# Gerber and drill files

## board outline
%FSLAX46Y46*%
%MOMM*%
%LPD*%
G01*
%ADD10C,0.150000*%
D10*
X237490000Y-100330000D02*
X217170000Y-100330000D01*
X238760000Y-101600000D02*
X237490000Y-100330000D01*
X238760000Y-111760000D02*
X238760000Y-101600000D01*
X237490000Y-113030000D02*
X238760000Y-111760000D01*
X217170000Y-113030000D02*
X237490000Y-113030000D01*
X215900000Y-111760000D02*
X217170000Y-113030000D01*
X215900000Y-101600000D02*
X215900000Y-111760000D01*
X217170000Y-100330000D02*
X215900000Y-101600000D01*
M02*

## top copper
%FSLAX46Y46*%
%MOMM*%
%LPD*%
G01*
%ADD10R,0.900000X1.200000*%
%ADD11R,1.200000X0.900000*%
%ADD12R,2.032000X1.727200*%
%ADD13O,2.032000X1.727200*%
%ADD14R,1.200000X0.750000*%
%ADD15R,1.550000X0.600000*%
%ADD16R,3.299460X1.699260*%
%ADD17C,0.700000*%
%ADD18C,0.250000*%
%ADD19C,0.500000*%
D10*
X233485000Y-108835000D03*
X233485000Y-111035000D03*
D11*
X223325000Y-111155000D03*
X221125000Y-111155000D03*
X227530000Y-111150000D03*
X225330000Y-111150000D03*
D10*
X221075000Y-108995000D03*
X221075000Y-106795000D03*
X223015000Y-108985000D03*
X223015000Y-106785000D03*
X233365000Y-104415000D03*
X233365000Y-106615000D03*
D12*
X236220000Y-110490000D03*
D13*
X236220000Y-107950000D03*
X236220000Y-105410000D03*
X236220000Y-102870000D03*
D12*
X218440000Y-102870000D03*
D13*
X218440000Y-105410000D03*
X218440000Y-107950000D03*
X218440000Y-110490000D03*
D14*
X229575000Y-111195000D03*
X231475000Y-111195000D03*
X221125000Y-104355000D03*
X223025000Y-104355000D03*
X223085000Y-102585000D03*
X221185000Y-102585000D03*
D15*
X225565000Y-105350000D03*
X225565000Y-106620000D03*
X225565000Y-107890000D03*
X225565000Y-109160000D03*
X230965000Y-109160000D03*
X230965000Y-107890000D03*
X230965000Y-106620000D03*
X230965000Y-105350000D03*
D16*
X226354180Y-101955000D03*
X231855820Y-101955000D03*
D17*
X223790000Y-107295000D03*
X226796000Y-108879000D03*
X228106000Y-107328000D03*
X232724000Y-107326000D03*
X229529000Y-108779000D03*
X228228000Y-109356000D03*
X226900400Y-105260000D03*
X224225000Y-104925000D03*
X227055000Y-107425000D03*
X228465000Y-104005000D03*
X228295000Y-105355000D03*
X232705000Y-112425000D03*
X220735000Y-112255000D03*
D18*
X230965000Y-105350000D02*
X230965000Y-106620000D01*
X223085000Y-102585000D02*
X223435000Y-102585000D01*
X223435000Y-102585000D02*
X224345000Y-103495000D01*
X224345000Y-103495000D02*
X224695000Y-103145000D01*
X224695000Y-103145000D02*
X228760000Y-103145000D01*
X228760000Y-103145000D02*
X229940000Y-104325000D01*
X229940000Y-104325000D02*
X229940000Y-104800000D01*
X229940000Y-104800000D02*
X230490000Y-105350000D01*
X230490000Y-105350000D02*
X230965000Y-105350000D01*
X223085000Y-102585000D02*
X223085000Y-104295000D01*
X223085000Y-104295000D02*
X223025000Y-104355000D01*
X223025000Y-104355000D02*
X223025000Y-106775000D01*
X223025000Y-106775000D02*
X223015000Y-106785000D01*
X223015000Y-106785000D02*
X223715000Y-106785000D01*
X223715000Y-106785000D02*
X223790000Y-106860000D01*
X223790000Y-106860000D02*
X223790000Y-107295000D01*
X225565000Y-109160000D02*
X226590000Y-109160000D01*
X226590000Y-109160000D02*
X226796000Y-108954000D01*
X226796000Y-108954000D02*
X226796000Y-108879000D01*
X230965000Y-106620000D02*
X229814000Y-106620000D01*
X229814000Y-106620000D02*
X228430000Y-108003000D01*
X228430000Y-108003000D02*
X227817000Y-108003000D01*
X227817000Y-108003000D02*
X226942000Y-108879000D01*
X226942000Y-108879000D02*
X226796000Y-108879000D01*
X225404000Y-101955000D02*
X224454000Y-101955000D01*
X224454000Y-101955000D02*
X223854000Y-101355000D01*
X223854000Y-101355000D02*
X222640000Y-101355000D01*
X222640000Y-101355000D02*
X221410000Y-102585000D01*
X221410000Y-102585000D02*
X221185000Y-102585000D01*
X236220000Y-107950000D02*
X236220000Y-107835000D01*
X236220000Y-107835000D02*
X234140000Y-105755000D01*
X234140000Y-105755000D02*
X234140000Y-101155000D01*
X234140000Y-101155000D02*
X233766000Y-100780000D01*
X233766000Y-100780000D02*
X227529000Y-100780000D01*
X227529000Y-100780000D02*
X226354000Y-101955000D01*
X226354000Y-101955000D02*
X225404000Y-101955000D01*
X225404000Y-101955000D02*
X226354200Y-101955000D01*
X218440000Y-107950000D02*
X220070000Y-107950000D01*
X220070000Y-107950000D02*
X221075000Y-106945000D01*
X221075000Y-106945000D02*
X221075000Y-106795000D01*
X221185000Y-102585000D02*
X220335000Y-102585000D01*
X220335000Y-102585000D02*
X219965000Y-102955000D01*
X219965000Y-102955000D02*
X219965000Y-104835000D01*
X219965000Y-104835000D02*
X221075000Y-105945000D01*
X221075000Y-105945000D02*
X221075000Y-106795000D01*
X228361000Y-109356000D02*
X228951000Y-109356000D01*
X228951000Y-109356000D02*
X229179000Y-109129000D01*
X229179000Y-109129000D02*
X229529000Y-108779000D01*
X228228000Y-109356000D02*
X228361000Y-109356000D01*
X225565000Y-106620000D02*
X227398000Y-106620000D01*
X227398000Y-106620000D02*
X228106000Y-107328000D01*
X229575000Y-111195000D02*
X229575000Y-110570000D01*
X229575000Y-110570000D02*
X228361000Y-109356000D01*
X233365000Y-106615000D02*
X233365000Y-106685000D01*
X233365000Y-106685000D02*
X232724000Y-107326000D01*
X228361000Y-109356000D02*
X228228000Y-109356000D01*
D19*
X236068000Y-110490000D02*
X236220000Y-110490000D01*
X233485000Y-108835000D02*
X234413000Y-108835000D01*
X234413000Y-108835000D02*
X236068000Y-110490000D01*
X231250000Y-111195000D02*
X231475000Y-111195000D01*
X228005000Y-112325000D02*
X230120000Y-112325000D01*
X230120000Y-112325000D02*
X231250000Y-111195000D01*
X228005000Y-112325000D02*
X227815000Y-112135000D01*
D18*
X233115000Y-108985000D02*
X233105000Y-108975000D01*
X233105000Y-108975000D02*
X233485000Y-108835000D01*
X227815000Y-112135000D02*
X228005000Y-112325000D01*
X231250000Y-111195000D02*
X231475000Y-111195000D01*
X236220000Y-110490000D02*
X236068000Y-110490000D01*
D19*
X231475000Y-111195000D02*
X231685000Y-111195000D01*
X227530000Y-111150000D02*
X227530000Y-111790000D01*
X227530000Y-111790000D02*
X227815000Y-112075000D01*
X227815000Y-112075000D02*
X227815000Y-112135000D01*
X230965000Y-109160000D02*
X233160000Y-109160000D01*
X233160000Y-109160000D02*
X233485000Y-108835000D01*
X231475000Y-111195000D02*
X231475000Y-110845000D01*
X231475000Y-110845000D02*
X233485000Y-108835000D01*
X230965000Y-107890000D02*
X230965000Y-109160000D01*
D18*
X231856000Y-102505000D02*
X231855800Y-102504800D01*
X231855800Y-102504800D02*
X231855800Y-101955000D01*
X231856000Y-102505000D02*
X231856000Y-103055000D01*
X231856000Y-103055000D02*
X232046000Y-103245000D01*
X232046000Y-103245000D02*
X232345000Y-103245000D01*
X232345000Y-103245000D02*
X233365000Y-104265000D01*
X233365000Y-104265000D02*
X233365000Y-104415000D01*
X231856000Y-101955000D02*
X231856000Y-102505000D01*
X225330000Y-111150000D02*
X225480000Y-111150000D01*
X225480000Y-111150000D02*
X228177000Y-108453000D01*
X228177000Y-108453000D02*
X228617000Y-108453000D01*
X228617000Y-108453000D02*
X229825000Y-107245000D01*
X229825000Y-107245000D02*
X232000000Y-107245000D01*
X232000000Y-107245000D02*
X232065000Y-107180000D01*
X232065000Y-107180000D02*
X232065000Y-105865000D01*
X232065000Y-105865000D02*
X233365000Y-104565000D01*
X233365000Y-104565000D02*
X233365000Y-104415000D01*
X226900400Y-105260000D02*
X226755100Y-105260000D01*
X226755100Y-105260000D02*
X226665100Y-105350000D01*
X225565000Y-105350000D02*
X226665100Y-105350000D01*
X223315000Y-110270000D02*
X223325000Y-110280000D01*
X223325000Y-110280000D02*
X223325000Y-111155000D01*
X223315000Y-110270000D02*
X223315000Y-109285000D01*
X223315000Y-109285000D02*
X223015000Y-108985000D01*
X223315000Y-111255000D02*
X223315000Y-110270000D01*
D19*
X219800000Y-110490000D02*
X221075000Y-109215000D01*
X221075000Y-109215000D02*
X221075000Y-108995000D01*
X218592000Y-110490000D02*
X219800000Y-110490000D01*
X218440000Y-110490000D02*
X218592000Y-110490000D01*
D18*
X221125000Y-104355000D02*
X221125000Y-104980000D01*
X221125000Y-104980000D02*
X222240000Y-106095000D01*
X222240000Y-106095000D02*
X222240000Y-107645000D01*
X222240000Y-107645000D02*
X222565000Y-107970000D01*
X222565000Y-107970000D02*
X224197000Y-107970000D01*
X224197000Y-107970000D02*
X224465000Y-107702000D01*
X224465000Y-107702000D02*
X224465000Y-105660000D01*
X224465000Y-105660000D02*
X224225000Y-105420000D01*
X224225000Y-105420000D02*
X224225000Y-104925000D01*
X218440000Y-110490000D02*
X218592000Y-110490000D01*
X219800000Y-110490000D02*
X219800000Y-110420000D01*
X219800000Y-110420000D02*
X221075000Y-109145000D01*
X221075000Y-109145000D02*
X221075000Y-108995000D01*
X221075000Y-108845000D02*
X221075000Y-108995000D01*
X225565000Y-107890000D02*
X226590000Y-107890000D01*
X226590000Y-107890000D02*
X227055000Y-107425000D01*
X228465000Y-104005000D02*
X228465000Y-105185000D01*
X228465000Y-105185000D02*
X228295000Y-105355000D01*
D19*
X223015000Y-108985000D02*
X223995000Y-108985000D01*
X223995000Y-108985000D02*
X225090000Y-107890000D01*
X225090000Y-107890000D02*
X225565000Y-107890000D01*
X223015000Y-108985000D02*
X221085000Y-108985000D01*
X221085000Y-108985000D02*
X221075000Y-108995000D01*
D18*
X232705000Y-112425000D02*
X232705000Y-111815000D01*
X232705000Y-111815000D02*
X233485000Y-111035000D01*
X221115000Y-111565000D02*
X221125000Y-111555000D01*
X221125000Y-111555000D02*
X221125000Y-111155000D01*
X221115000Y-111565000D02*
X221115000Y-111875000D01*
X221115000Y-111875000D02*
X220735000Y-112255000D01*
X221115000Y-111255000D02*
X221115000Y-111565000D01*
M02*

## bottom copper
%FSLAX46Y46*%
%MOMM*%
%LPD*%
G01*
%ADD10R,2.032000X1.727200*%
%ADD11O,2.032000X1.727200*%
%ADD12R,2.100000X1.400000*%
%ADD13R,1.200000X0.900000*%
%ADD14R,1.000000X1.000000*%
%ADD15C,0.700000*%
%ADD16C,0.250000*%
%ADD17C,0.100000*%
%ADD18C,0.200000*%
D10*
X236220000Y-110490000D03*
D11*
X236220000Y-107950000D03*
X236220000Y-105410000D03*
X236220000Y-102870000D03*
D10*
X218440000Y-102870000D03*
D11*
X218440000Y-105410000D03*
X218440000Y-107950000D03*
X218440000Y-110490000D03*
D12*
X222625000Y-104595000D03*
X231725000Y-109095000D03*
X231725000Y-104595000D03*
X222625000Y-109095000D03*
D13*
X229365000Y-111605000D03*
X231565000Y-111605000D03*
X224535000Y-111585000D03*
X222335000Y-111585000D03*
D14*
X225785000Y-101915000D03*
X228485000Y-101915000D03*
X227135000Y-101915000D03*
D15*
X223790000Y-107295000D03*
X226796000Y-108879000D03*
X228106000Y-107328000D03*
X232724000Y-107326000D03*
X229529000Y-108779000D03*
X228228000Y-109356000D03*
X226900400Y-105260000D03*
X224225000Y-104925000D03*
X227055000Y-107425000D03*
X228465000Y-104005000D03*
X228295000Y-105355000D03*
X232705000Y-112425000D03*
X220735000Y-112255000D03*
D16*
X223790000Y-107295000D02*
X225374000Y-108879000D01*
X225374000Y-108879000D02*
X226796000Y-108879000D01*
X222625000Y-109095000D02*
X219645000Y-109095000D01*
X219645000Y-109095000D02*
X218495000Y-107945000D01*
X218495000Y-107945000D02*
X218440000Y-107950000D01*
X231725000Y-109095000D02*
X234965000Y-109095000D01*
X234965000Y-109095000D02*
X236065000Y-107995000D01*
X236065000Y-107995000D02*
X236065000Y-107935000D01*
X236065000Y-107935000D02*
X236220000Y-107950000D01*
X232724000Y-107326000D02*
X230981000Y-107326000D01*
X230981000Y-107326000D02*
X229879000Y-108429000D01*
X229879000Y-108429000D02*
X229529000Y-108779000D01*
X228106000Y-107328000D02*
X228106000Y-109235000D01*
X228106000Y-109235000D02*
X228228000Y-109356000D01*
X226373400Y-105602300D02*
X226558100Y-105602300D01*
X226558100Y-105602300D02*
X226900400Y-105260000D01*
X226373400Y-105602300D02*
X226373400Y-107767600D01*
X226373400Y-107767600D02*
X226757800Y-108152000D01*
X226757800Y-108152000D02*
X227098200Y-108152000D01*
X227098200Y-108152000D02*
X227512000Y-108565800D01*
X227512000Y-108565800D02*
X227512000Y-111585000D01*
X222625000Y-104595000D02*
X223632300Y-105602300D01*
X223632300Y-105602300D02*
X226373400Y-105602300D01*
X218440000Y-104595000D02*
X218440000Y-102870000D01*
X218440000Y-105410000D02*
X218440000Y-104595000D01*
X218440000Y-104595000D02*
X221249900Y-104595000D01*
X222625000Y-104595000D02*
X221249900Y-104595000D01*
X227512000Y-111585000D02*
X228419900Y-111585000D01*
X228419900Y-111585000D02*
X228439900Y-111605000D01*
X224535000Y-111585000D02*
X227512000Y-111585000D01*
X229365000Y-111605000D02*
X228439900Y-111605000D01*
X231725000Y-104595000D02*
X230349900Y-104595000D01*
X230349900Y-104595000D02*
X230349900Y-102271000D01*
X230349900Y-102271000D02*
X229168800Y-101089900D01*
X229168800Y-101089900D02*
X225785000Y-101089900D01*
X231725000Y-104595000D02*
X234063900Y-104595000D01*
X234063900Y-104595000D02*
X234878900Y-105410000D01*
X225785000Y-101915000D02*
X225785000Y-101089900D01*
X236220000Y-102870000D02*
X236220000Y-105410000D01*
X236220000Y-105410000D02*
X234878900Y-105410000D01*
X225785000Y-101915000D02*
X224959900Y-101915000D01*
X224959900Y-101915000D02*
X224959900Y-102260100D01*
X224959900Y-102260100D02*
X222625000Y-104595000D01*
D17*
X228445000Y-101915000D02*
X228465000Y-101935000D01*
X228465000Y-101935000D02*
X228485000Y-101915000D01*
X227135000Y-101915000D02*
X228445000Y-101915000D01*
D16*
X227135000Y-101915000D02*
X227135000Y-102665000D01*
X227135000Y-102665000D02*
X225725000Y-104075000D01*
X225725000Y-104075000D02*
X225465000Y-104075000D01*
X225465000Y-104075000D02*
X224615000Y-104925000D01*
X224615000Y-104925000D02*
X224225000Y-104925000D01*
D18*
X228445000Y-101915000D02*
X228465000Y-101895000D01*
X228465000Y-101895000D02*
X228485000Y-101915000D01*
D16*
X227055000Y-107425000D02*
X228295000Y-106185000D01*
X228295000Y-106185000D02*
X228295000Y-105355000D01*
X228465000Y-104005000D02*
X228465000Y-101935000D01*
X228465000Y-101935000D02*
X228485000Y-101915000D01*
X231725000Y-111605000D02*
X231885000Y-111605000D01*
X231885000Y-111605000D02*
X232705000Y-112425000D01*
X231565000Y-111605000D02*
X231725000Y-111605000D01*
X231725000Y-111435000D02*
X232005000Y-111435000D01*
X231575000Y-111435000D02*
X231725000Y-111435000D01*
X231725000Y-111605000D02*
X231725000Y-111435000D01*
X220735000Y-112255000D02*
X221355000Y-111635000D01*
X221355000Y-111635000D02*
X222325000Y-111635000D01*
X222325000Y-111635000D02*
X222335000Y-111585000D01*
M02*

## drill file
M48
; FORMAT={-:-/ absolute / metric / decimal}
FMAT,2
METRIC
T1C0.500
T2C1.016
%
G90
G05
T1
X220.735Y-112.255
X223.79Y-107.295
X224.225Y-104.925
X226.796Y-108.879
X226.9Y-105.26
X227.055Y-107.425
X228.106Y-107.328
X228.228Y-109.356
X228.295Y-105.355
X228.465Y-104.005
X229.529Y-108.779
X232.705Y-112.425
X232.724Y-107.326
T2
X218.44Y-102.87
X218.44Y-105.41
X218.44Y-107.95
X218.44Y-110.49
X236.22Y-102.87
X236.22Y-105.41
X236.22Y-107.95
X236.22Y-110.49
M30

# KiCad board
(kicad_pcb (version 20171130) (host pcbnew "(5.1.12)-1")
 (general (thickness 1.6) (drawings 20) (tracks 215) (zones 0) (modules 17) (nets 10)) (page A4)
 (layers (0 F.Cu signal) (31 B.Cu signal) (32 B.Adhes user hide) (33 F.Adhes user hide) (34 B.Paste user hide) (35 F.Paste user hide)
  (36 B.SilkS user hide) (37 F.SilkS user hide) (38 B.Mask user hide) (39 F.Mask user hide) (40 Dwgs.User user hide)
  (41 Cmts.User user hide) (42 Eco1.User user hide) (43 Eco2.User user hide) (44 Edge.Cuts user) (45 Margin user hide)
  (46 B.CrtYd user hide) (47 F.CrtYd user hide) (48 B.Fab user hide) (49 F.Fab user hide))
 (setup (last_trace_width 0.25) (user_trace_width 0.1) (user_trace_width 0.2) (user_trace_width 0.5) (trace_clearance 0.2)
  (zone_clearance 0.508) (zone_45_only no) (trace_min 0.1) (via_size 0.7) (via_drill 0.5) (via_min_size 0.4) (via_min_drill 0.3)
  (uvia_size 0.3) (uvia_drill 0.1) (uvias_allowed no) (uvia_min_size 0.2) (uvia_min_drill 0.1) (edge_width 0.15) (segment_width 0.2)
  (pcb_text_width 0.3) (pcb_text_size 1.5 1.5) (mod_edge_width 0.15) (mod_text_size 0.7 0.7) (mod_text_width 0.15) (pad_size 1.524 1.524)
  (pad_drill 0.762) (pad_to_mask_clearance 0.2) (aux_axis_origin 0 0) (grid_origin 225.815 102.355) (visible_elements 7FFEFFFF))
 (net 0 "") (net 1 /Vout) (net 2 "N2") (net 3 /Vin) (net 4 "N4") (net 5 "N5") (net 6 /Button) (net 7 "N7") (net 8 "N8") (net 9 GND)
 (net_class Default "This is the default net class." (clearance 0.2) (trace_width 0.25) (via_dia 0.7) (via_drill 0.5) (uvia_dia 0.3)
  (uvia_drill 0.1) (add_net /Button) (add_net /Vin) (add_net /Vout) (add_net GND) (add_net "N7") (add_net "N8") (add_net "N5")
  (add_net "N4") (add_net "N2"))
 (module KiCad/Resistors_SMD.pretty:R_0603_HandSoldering (layer F.Cu) (at 233.485 109.935 270)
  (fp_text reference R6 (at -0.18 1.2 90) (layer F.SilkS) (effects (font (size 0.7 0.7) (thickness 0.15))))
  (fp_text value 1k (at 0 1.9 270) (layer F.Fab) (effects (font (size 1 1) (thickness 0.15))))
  (pad 1 smd rect (at -1.1 0 270) (size 1.2 0.9) (layers F.Cu F.Paste F.Mask) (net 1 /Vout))
  (pad 2 smd rect (at 1.1 0 270) (size 1.2 0.9) (layers F.Cu F.Paste F.Mask) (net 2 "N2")))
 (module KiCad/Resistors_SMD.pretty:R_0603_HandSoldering (layer F.Cu) (at 222.225 111.155 180)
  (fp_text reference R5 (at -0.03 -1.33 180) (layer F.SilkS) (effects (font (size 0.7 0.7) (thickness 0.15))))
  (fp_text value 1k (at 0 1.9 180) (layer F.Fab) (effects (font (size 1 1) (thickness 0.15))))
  (pad 1 smd rect (at -1.1 0 180) (size 1.2 0.9) (layers F.Cu F.Paste F.Mask) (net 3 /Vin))
  (pad 2 smd rect (at 1.1 0 180) (size 1.2 0.9) (layers F.Cu F.Paste F.Mask) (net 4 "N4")))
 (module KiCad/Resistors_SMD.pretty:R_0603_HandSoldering (layer F.Cu) (at 226.43 111.15 180)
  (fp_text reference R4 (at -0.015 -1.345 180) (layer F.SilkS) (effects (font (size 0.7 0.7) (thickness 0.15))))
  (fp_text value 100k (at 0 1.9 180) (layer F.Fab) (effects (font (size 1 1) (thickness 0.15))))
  (pad 1 smd rect (at -1.1 0 180) (size 1.2 0.9) (layers F.Cu F.Paste F.Mask) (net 1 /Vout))
  (pad 2 smd rect (at 1.1 0 180) (size 1.2 0.9) (layers F.Cu F.Paste F.Mask) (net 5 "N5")))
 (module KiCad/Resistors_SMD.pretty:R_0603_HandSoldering (layer F.Cu) (at 221.075 107.895 90)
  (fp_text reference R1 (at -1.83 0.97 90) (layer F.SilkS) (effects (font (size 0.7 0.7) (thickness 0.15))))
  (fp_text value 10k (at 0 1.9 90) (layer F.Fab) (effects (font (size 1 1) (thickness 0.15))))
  (pad 1 smd rect (at -1.1 0 90) (size 1.2 0.9) (layers F.Cu F.Paste F.Mask) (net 3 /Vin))
  (pad 2 smd rect (at 1.1 0 90) (size 1.2 0.9) (layers F.Cu F.Paste F.Mask) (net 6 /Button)))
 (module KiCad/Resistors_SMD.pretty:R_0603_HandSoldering (layer F.Cu) (at 223.015 107.885 90)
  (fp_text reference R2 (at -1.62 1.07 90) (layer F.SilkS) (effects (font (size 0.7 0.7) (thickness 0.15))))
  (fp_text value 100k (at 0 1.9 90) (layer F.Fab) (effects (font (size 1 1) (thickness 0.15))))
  (pad 1 smd rect (at -1.1 0 90) (size 1.2 0.9) (layers F.Cu F.Paste F.Mask) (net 3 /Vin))
  (pad 2 smd rect (at 1.1 0 90) (size 1.2 0.9) (layers F.Cu F.Paste F.Mask) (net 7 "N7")))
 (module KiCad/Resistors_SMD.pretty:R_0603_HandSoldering (layer F.Cu) (at 233.365 105.515 270)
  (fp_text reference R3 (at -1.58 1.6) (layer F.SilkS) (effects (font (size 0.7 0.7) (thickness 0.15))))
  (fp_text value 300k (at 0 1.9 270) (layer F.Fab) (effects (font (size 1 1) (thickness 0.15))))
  (pad 1 smd rect (at -1.1 0 270) (size 1.2 0.9) (layers F.Cu F.Paste F.Mask) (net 5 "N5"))
  (pad 2 smd rect (at 1.1 0 270) (size 1.2 0.9) (layers F.Cu F.Paste F.Mask) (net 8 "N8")))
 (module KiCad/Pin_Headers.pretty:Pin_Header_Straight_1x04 (layer F.Cu) (at 236.22 110.49 180)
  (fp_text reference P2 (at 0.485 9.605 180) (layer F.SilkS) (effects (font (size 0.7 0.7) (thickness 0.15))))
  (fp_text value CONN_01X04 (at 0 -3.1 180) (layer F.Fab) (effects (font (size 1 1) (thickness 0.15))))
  (pad 1 thru_hole rect (at 0 0 180) (size 2.032 1.7272) (drill 1.016) (layers *.Cu *.Mask F.SilkS) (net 1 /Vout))
  (pad 2 thru_hole oval (at 0 2.54 180) (size 2.032 1.7272) (drill 1.016) (layers *.Cu *.Mask F.SilkS) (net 6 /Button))
  (pad 3 thru_hole oval (at 0 5.08 180) (size 2.032 1.7272) (drill 1.016) (layers *.Cu *.Mask F.SilkS) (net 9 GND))
  (pad 4 thru_hole oval (at 0 7.62 180) (size 2.032 1.7272) (drill 1.016) (layers *.Cu *.Mask F.SilkS) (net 9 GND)))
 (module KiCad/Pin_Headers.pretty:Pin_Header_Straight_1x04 (layer F.Cu) (at 218.44 102.87)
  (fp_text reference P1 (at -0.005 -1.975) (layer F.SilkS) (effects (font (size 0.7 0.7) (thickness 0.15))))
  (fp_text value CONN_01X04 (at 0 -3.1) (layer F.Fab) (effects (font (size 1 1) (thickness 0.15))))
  (pad 1 thru_hole rect (at 0 0) (size 2.032 1.7272) (drill 1.016) (layers *.Cu *.Mask F.SilkS) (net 9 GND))
  (pad 2 thru_hole oval (at 0 2.54) (size 2.032 1.7272) (drill 1.016) (layers *.Cu *.Mask F.SilkS) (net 9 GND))
  (pad 3 thru_hole oval (at 0 5.08) (size 2.032 1.7272) (drill 1.016) (layers *.Cu *.Mask F.SilkS) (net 6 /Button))
  (pad 4 thru_hole oval (at 0 7.62) (size 2.032 1.7272) (drill 1.016) (layers *.Cu *.Mask F.SilkS) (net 3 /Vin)))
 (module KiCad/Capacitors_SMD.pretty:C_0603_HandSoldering (layer F.Cu) (at 230.525 111.195)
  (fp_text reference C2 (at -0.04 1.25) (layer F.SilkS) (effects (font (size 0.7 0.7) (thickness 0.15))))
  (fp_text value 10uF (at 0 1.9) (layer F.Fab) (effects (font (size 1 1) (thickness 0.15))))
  (pad 1 smd rect (at -0.95 0) (size 1.2 0.75) (layers F.Cu F.Paste F.Mask) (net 8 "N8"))
  (pad 2 smd rect (at 0.95 0) (size 1.2 0.75) (layers F.Cu F.Paste F.Mask) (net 1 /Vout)))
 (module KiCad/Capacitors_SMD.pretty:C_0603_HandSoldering (layer F.Cu) (at 222.075 104.355)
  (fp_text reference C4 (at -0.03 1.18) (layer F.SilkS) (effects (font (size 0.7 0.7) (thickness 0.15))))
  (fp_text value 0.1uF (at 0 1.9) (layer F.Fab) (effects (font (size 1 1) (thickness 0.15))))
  (pad 1 smd rect (at -0.95 0) (size 1.2 0.75) (layers F.Cu F.Paste F.Mask) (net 3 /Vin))
  (pad 2 smd rect (at 0.95 0) (size 1.2 0.75) (layers F.Cu F.Paste F.Mask) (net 7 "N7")))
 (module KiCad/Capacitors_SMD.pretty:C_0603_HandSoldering (layer F.Cu) (at 222.135 102.585 180)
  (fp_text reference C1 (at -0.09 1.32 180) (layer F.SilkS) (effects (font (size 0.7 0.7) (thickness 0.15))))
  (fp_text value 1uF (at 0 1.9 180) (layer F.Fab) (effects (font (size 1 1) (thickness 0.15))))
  (pad 1 smd rect (at -0.95 0 180) (size 1.2 0.75) (layers F.Cu F.Paste F.Mask) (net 7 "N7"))
  (pad 2 smd rect (at 0.95 0 180) (size 1.2 0.75) (layers F.Cu F.Paste F.Mask) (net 6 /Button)))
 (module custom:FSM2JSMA (layer B.Cu) (at 227.175 106.845 270)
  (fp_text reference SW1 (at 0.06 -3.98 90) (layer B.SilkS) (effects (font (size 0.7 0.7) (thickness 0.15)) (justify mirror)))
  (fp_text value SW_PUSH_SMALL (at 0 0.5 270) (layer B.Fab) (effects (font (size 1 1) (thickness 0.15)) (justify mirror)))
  (pad 2 smd rect (at -2.25 4.55 270) (size 1.4 2.1) (layers B.Cu B.Paste B.Mask) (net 9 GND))
  (pad 1 smd rect (at 2.25 -4.55 270) (size 1.4 2.1) (layers B.Cu B.Paste B.Mask) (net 6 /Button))
  (pad 2 smd rect (at -2.25 -4.55 270) (size 1.4 2.1) (layers B.Cu B.Paste B.Mask) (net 9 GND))
  (pad 1 smd rect (at 2.25 4.55 270) (size 1.4 2.1) (layers B.Cu B.Paste B.Mask) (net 6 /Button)))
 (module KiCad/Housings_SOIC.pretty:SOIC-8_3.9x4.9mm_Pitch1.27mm (layer F.Cu) (at 228.265 107.255)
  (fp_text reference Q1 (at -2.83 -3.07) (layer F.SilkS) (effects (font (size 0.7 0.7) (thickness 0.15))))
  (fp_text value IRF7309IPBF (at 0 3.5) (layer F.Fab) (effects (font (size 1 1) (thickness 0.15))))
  (pad 1 smd rect (at -2.7 -1.905) (size 1.55 0.6) (layers F.Cu F.Paste F.Mask) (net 9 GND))
  (pad 2 smd rect (at -2.7 -0.635) (size 1.55 0.6) (layers F.Cu F.Paste F.Mask) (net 8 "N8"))
  (pad 3 smd rect (at -2.7 0.635) (size 1.55 0.6) (layers F.Cu F.Paste F.Mask) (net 3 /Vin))
  (pad 4 smd rect (at -2.7 1.905) (size 1.55 0.6) (layers F.Cu F.Paste F.Mask) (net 7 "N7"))
  (pad 5 smd rect (at 2.7 1.905) (size 1.55 0.6) (layers F.Cu F.Paste F.Mask) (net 1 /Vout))
  (pad 6 smd rect (at 2.7 0.635) (size 1.55 0.6) (layers F.Cu F.Paste F.Mask) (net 1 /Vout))
  (pad 7 smd rect (at 2.7 -0.635) (size 1.55 0.6) (layers F.Cu F.Paste F.Mask) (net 7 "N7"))
  (pad 8 smd rect (at 2.7 -1.905) (size 1.55 0.6) (layers F.Cu F.Paste F.Mask) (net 7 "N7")))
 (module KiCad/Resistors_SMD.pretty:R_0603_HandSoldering (layer B.Cu) (at 230.465 111.605)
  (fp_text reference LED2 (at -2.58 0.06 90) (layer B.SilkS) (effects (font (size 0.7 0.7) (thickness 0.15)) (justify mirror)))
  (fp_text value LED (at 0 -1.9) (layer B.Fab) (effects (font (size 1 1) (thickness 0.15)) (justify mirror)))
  (pad 1 smd rect (at -1.1 0) (size 1.2 0.9) (layers B.Cu B.Paste B.Mask) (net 9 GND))
  (pad 2 smd rect (at 1.1 0) (size 1.2 0.9) (layers B.Cu B.Paste B.Mask) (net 2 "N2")))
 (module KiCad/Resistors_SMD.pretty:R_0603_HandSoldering (layer B.Cu) (at 223.435 111.585 180)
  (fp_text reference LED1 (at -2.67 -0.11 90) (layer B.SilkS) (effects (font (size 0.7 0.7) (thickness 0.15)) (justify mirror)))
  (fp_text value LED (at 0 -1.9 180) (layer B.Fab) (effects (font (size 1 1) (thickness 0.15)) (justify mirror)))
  (pad 1 smd rect (at -1.1 0 180) (size 1.2 0.9) (layers B.Cu B.Paste B.Mask) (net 9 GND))
  (pad 2 smd rect (at 1.1 0 180) (size 1.2 0.9) (layers B.Cu B.Paste B.Mask) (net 4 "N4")))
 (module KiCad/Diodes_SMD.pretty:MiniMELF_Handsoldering (layer F.Cu) (at 229.105 101.955)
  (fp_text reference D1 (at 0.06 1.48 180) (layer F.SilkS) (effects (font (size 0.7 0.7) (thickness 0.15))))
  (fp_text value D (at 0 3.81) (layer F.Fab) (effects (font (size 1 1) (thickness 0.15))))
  (pad 1 smd rect (at -2.75082 0) (size 3.29946 1.69926) (layers F.Cu F.Paste F.Mask) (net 6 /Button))
  (pad 2 smd rect (at 2.75082 0) (size 3.29946 1.69926) (layers F.Cu F.Paste F.Mask) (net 5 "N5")))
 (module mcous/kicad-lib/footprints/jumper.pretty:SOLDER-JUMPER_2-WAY (layer B.Cu) (at 227.135 101.915)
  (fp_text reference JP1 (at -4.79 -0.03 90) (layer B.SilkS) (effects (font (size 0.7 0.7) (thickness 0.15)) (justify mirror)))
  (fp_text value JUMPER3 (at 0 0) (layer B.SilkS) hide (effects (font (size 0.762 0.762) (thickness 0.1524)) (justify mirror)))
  (pad 1 smd rect (at -1.35 0) (size 1 1) (layers B.Cu B.Paste B.Mask) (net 9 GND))
  (pad 3 smd rect (at 1.35 0) (size 1 1) (layers B.Cu B.Paste B.Mask) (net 3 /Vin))
  (pad 2 smd rect (at 0 0) (size 1 1) (layers B.Cu B.Paste B.Mask) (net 3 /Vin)))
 (gr_line (start 237.49 100.33) (end 217.17 100.33) (angle 90) (layer Edge.Cuts) (width 0.15))
 (gr_line (start 238.76 101.6) (end 237.49 100.33) (angle 90) (layer Edge.Cuts) (width 0.15))
 (gr_line (start 238.76 111.76) (end 238.76 101.6) (angle 90) (layer Edge.Cuts) (width 0.15))
 (gr_line (start 237.49 113.03) (end 238.76 111.76) (angle 90) (layer Edge.Cuts) (width 0.15))
 (gr_line (start 217.17 113.03) (end 237.49 113.03) (angle 90) (layer Edge.Cuts) (width 0.15))
 (gr_line (start 215.9 111.76) (end 217.17 113.03) (angle 90) (layer Edge.Cuts) (width 0.15))
 (gr_line (start 215.9 101.6) (end 215.9 111.76) (angle 90) (layer Edge.Cuts) (width 0.15))
 (gr_line (start 217.17 100.33) (end 215.9 101.6) (angle 90) (layer Edge.Cuts) (width 0.15))
 (segment (start 230.965 105.35) (end 230.965 106.62) (width 0.25) (layer F.Cu) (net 7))
 (segment (start 223.085 102.585) (end 223.435 102.585) (width 0.25) (layer F.Cu) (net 7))
 (segment (start 223.435 102.585) (end 224.345 103.495) (width 0.25) (layer F.Cu) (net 7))
 (segment (start 224.345 103.495) (end 224.695 103.145) (width 0.25) (layer F.Cu) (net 7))
 (segment (start 224.695 103.145) (end 228.76 103.145) (width 0.25) (layer F.Cu) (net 7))
 (segment (start 228.76 103.145) (end 229.94 104.325) (width 0.25) (layer F.Cu) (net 7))
 (segment (start 229.94 104.325) (end 229.94 104.8) (width 0.25) (layer F.Cu) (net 7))
 (segment (start 229.94 104.8) (end 230.49 105.35) (width 0.25) (layer F.Cu) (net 7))
 (segment (start 230.49 105.35) (end 230.965 105.35) (width 0.25) (layer F.Cu) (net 7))
 (segment (start 223.085 102.585) (end 223.085 104.295) (width 0.25) (layer F.Cu) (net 7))
 (segment (start 223.085 104.295) (end 223.025 104.355) (width 0.25) (layer F.Cu) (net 7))
 (segment (start 223.025 104.355) (end 223.025 106.775) (width 0.25) (layer F.Cu) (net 7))
 (segment (start 223.025 106.775) (end 223.015 106.785) (width 0.25) (layer F.Cu) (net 7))
 (segment (start 223.015 106.785) (end 223.715 106.785) (width 0.25) (layer F.Cu) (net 7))
 (segment (start 223.715 106.785) (end 223.79 106.86) (width 0.25) (layer F.Cu) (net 7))
 (segment (start 223.79 106.86) (end 223.79 107.295) (width 0.25) (layer F.Cu) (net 7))
 (segment (start 225.565 109.16) (end 226.59 109.16) (width 0.25) (layer F.Cu) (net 7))
 (segment (start 226.59 109.16) (end 226.796 108.954) (width 0.25) (layer F.Cu) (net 7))
 (segment (start 226.796 108.954) (end 226.796 108.879) (width 0.25) (layer F.Cu) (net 7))
 (segment (start 223.79 107.295) (end 225.374 108.879) (width 0.25) (layer B.Cu) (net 7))
 (segment (start 225.374 108.879) (end 226.796 108.879) (width 0.25) (layer B.Cu) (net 7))
 (segment (start 230.965 106.62) (end 229.814 106.62) (width 0.25) (layer F.Cu) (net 7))
 (segment (start 229.814 106.62) (end 228.43 108.003) (width 0.25) (layer F.Cu) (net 7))
 (segment (start 228.43 108.003) (end 227.817 108.003) (width 0.25) (layer F.Cu) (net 7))
 (segment (start 227.817 108.003) (end 226.942 108.879) (width 0.25) (layer F.Cu) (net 7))
 (segment (start 226.942 108.879) (end 226.796 108.879) (width 0.25) (layer F.Cu) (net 7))
 (via (at 223.79 107.295) (size 0.7) (layers F.Cu B.Cu) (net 7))
 (via (at 226.796 108.879) (size 0.7) (layers F.Cu B.Cu) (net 7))
 (segment (start 225.404 101.955) (end 224.454 101.955) (width 0.25) (layer F.Cu) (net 6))
 (segment (start 224.454 101.955) (end 223.854 101.355) (width 0.25) (layer F.Cu) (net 6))
 (segment (start 223.854 101.355) (end 222.64 101.355) (width 0.25) (layer F.Cu) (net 6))
 (segment (start 222.64 101.355) (end 221.41 102.585) (width 0.25) (layer F.Cu) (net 6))
 (segment (start 221.41 102.585) (end 221.185 102.585) (width 0.25) (layer F.Cu) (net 6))
 (segment (start 236.22 107.95) (end 236.22 107.835) (width 0.25) (layer F.Cu) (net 6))
 (segment (start 236.22 107.835) (end 234.14 105.755) (width 0.25) (layer F.Cu) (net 6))
 (segment (start 234.14 105.755) (end 234.14 101.155) (width 0.25) (layer F.Cu) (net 6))
 (segment (start 234.14 101.155) (end 233.766 100.78) (width 0.25) (layer F.Cu) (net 6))
 (segment (start 233.766 100.78) (end 227.529 100.78) (width 0.25) (layer F.Cu) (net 6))
 (segment (start 227.529 100.78) (end 226.354 101.955) (width 0.25) (layer F.Cu) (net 6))
 (segment (start 226.354 101.955) (end 225.404 101.955) (width 0.25) (layer F.Cu) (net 6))
 (segment (start 225.404 101.955) (end 226.3542 101.955) (width 0.25) (layer F.Cu) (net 6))
 (segment (start 218.44 107.95) (end 220.07 107.95) (width 0.25) (layer F.Cu) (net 6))
 (segment (start 220.07 107.95) (end 221.075 106.945) (width 0.25) (layer F.Cu) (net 6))
 (segment (start 221.075 106.945) (end 221.075 106.795) (width 0.25) (layer F.Cu) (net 6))
 (segment (start 222.625 109.095) (end 219.645 109.095) (width 0.25) (layer B.Cu) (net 6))
 (segment (start 219.645 109.095) (end 218.495 107.945) (width 0.25) (layer B.Cu) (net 6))
 (segment (start 218.495 107.945) (end 218.44 107.95) (width 0.25) (layer B.Cu) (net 6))
 (segment (start 231.725 109.095) (end 234.965 109.095) (width 0.25) (layer B.Cu) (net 6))
 (segment (start 234.965 109.095) (end 236.065 107.995) (width 0.25) (layer B.Cu) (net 6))
 (segment (start 236.065 107.995) (end 236.065 107.935) (width 0.25) (layer B.Cu) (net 6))
 (segment (start 236.065 107.935) (end 236.22 107.95) (width 0.25) (layer B.Cu) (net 6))
 (segment (start 221.185 102.585) (end 220.335 102.585) (width 0.25) (layer F.Cu) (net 6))
 (segment (start 220.335 102.585) (end 219.965 102.955) (width 0.25) (layer F.Cu) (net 6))
 (segment (start 219.965 102.955) (end 219.965 104.835) (width 0.25) (layer F.Cu) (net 6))
 (segment (start 219.965 104.835) (end 221.075 105.945) (width 0.25) (layer F.Cu) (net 6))
 (segment (start 221.075 105.945) (end 221.075 106.795) (width 0.25) (layer F.Cu) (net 6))
 (segment (start 228.361 109.356) (end 228.951 109.356) (width 0.25) (layer F.Cu) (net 8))
 (segment (start 228.951 109.356) (end 229.179 109.129) (width 0.25) (layer F.Cu) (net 8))
 (segment (start 229.179 109.129) (end 229.529 108.779) (width 0.25) (layer F.Cu) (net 8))
 (segment (start 228.228 109.356) (end 228.361 109.356) (width 0.25) (layer F.Cu) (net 8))
 (segment (start 225.565 106.62) (end 227.398 106.62) (width 0.25) (layer F.Cu) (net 8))
 (segment (start 227.398 106.62) (end 228.106 107.328) (width 0.25) (layer F.Cu) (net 8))
 (segment (start 232.724 107.326) (end 230.981 107.326) (width 0.25) (layer B.Cu) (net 8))
 (segment (start 230.981 107.326) (end 229.879 108.429) (width 0.25) (layer B.Cu) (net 8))
 (segment (start 229.879 108.429) (end 229.529 108.779) (width 0.25) (layer B.Cu) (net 8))
 (segment (start 229.575 111.195) (end 229.575 110.57) (width 0.25) (layer F.Cu) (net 8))
 (segment (start 229.575 110.57) (end 228.361 109.356) (width 0.25) (layer F.Cu) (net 8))
 (segment (start 233.365 106.615) (end 233.365 106.685) (width 0.25) (layer F.Cu) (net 8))
 (segment (start 233.365 106.685) (end 232.724 107.326) (width 0.25) (layer F.Cu) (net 8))
 (segment (start 228.106 107.328) (end 228.106 109.235) (width 0.25) (layer B.Cu) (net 8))
 (segment (start 228.106 109.235) (end 228.228 109.356) (width 0.25) (layer B.Cu) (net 8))
 (segment (start 228.361 109.356) (end 228.228 109.356) (width 0.25) (layer F.Cu) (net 8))
 (via (at 228.106 107.328) (size 0.7) (layers F.Cu B.Cu) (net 8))
 (via (at 232.724 107.326) (size 0.7) (layers F.Cu B.Cu) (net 8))
 (via (at 229.529 108.779) (size 0.7) (layers F.Cu B.Cu) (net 8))
 (via (at 228.228 109.356) (size 0.7) (layers F.Cu B.Cu) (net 8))
 (segment (start 236.068 110.49) (end 236.22 110.49) (width 0.5) (layer F.Cu) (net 1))
 (segment (start 233.485 108.835) (end 234.413 108.835) (width 0.5) (layer F.Cu) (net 1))
 (segment (start 234.413 108.835) (end 236.068 110.49) (width 0.5) (layer F.Cu) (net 1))
 (segment (start 231.25 111.195) (end 231.475 111.195) (width 0.5) (layer F.Cu) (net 1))
 (segment (start 228.005 112.325) (end 230.12 112.325) (width 0.5) (layer F.Cu) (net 1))
 (segment (start 230.12 112.325) (end 231.25 111.195) (width 0.5) (layer F.Cu) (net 1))
 (segment (start 228.005 112.325) (end 227.815 112.135) (width 0.5) (layer F.Cu) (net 1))
 (segment (start 233.115 108.985) (end 233.105 108.975) (width 0.25) (layer F.Cu) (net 1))
 (segment (start 233.105 108.975) (end 233.485 108.835) (width 0.25) (layer F.Cu) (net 1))
 (segment (start 227.815 112.135) (end 228.005 112.325) (width 0.25) (layer F.Cu) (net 1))
 (segment (start 231.25 111.195) (end 231.475 111.195) (width 0.25) (layer F.Cu) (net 1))
 (segment (start 236.22 110.49) (end 236.068 110.49) (width 0.25) (layer F.Cu) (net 1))
 (segment (start 231.475 111.195) (end 231.685 111.195) (width 0.5) (layer F.Cu) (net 1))
 (segment (start 227.53 111.15) (end 227.53 111.79) (width 0.5) (layer F.Cu) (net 1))
 (segment (start 227.53 111.79) (end 227.815 112.075) (width 0.5) (layer F.Cu) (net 1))
 (segment (start 227.815 112.075) (end 227.815 112.135) (width 0.5) (layer F.Cu) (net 1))
 (segment (start 230.965 109.16) (end 233.16 109.16) (width 0.5) (layer F.Cu) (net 1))
 (segment (start 233.16 109.16) (end 233.485 108.835) (width 0.5) (layer F.Cu) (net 1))
 (segment (start 231.475 111.195) (end 231.475 110.845) (width 0.5) (layer F.Cu) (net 1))
 (segment (start 231.475 110.845) (end 233.485 108.835) (width 0.5) (layer F.Cu) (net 1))
 (segment (start 230.965 107.89) (end 230.965 109.16) (width 0.5) (layer F.Cu) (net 1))
 (segment (start 231.856 102.505) (end 231.8558 102.5048) (width 0.25) (layer F.Cu) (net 5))
 (segment (start 231.8558 102.5048) (end 231.8558 101.955) (width 0.25) (layer F.Cu) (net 5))
 (segment (start 231.856 102.505) (end 231.856 103.055) (width 0.25) (layer F.Cu) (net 5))
 (segment (start 231.856 103.055) (end 232.046 103.245) (width 0.25) (layer F.Cu) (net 5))
 (segment (start 232.046 103.245) (end 232.345 103.245) (width 0.25) (layer F.Cu) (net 5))
 (segment (start 232.345 103.245) (end 233.365 104.265) (width 0.25) (layer F.Cu) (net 5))
 (segment (start 233.365 104.265) (end 233.365 104.415) (width 0.25) (layer F.Cu) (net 5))
 (segment (start 231.856 101.955) (end 231.856 102.505) (width 0.25) (layer F.Cu) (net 5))
 (segment (start 225.33 111.15) (end 225.48 111.15) (width 0.25) (layer F.Cu) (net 5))
 (segment (start 225.48 111.15) (end 228.177 108.453) (width 0.25) (layer F.Cu) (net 5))
 (segment (start 228.177 108.453) (end 228.617 108.453) (width 0.25) (layer F.Cu) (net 5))
 (segment (start 228.617 108.453) (end 229.825 107.245) (width 0.25) (layer F.Cu) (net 5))
 (segment (start 229.825 107.245) (end 232 107.245) (width 0.25) (layer F.Cu) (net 5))
 (segment (start 232 107.245) (end 232.065 107.18) (width 0.25) (layer F.Cu) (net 5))
 (segment (start 232.065 107.18) (end 232.065 105.865) (width 0.25) (layer F.Cu) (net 5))
 (segment (start 232.065 105.865) (end 233.365 104.565) (width 0.25) (layer F.Cu) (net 5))
 (segment (start 233.365 104.565) (end 233.365 104.415) (width 0.25) (layer F.Cu) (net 5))
 (segment (start 226.9004 105.26) (end 226.7551 105.26) (width 0.25) (layer F.Cu) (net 9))
 (segment (start 226.7551 105.26) (end 226.6651 105.35) (width 0.25) (layer F.Cu) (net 9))
 (segment (start 226.3734 105.6023) (end 226.5581 105.6023) (width 0.25) (layer B.Cu) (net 9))
 (segment (start 226.5581 105.6023) (end 226.9004 105.26) (width 0.25) (layer B.Cu) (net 9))
 (segment (start 225.565 105.35) (end 226.6651 105.35) (width 0.25) (layer F.Cu) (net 9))
 (segment (start 226.3734 105.6023) (end 226.3734 107.7676) (width 0.25) (layer B.Cu) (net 9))
 (segment (start 226.3734 107.7676) (end 226.7578 108.152) (width 0.25) (layer B.Cu) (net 9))
 (segment (start 226.7578 108.152) (end 227.0982 108.152) (width 0.25) (layer B.Cu) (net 9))
 (segment (start 227.0982 108.152) (end 227.512 108.5658) (width 0.25) (layer B.Cu) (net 9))
 (segment (start 227.512 108.5658) (end 227.512 111.585) (width 0.25) (layer B.Cu) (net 9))
 (segment (start 222.625 104.595) (end 223.6323 105.6023) (width 0.25) (layer B.Cu) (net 9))
 (segment (start 223.6323 105.6023) (end 226.3734 105.6023) (width 0.25) (layer B.Cu) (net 9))
 (segment (start 218.44 104.595) (end 218.44 102.87) (width 0.25) (layer B.Cu) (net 9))
 (segment (start 218.44 105.41) (end 218.44 104.595) (width 0.25) (layer B.Cu) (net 9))
 (segment (start 218.44 104.595) (end 221.2499 104.595) (width 0.25) (layer B.Cu) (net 9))
 (segment (start 222.625 104.595) (end 221.2499 104.595) (width 0.25) (layer B.Cu) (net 9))
 (segment (start 227.512 111.585) (end 228.4199 111.585) (width 0.25) (layer B.Cu) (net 9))
 (segment (start 228.4199 111.585) (end 228.4399 111.605) (width 0.25) (layer B.Cu) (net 9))
 (segment (start 224.535 111.585) (end 227.512 111.585) (width 0.25) (layer B.Cu) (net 9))
 (segment (start 229.365 111.605) (end 228.4399 111.605) (width 0.25) (layer B.Cu) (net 9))
 (segment (start 231.725 104.595) (end 230.3499 104.595) (width 0.25) (layer B.Cu) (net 9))
 (segment (start 230.3499 104.595) (end 230.3499 102.271) (width 0.25) (layer B.Cu) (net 9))
 (segment (start 230.3499 102.271) (end 229.1688 101.0899) (width 0.25) (layer B.Cu) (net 9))
 (segment (start 229.1688 101.0899) (end 225.785 101.0899) (width 0.25) (layer B.Cu) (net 9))
 (segment (start 231.725 104.595) (end 234.0639 104.595) (width 0.25) (layer B.Cu) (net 9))
 (segment (start 234.0639 104.595) (end 234.8789 105.41) (width 0.25) (layer B.Cu) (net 9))
 (segment (start 225.785 101.915) (end 225.785 101.0899) (width 0.25) (layer B.Cu) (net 9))
 (segment (start 236.22 102.87) (end 236.22 105.41) (width 0.25) (layer B.Cu) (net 9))
 (segment (start 236.22 105.41) (end 234.8789 105.41) (width 0.25) (layer B.Cu) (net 9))
 (segment (start 225.785 101.915) (end 224.9599 101.915) (width 0.25) (layer B.Cu) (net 9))
 (segment (start 224.9599 101.915) (end 224.9599 102.2601) (width 0.25) (layer B.Cu) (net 9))
 (segment (start 224.9599 102.2601) (end 222.625 104.595) (width 0.25) (layer B.Cu) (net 9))
 (via (at 226.9004 105.26) (size 0.7) (layers F.Cu B.Cu) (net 9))
 (segment (start 223.315 110.27) (end 223.325 110.28) (width 0.25) (layer F.Cu) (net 3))
 (segment (start 223.325 110.28) (end 223.325 111.155) (width 0.25) (layer F.Cu) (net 3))
 (segment (start 223.315 110.27) (end 223.315 109.285) (width 0.25) (layer F.Cu) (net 3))
 (segment (start 223.315 109.285) (end 223.015 108.985) (width 0.25) (layer F.Cu) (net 3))
 (segment (start 223.315 111.255) (end 223.315 110.27) (width 0.25) (layer F.Cu) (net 3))
 (segment (start 228.445 101.915) (end 228.465 101.935) (width 0.1) (layer B.Cu) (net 3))
 (segment (start 228.465 101.935) (end 228.485 101.915) (width 0.1) (layer B.Cu) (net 3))
 (segment (start 227.135 101.915) (end 228.445 101.915) (width 0.1) (layer B.Cu) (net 3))
 (segment (start 219.8 110.49) (end 221.075 109.215) (width 0.5) (layer F.Cu) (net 3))
 (segment (start 221.075 109.215) (end 221.075 108.995) (width 0.5) (layer F.Cu) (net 3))
 (segment (start 218.592 110.49) (end 219.8 110.49) (width 0.5) (layer F.Cu) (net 3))
 (segment (start 218.44 110.49) (end 218.592 110.49) (width 0.5) (layer F.Cu) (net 3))
 (segment (start 227.135 101.915) (end 227.135 102.665) (width 0.25) (layer B.Cu) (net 3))
 (segment (start 227.135 102.665) (end 225.725 104.075) (width 0.25) (layer B.Cu) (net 3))
 (segment (start 225.725 104.075) (end 225.465 104.075) (width 0.25) (layer B.Cu) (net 3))
 (segment (start 225.465 104.075) (end 224.615 104.925) (width 0.25) (layer B.Cu) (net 3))
 (segment (start 224.615 104.925) (end 224.225 104.925) (width 0.25) (layer B.Cu) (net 3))
 (segment (start 221.125 104.355) (end 221.125 104.98) (width 0.25) (layer F.Cu) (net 3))
 (segment (start 221.125 104.98) (end 222.24 106.095) (width 0.25) (layer F.Cu) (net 3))
 (segment (start 222.24 106.095) (end 222.24 107.645) (width 0.25) (layer F.Cu) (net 3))
 (segment (start 222.24 107.645) (end 222.565 107.97) (width 0.25) (layer F.Cu) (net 3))
 (segment (start 222.565 107.97) (end 224.197 107.97) (width 0.25) (layer F.Cu) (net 3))
 (segment (start 224.197 107.97) (end 224.465 107.702) (width 0.25) (layer F.Cu) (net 3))
 (segment (start 224.465 107.702) (end 224.465 105.66) (width 0.25) (layer F.Cu) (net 3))
 (segment (start 224.465 105.66) (end 224.225 105.42) (width 0.25) (layer F.Cu) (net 3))
 (segment (start 224.225 105.42) (end 224.225 104.925) (width 0.25) (layer F.Cu) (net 3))
 (segment (start 218.44 110.49) (end 218.592 110.49) (width 0.25) (layer F.Cu) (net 3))
 (segment (start 219.8 110.49) (end 219.8 110.42) (width 0.25) (layer F.Cu) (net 3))
 (segment (start 219.8 110.42) (end 221.075 109.145) (width 0.25) (layer F.Cu) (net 3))
 (segment (start 221.075 109.145) (end 221.075 108.995) (width 0.25) (layer F.Cu) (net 3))
 (segment (start 221.075 108.845) (end 221.075 108.995) (width 0.25) (layer F.Cu) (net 3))
 (segment (start 228.445 101.915) (end 228.465 101.895) (width 0.2) (layer B.Cu) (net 3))
 (segment (start 228.465 101.895) (end 228.485 101.915) (width 0.2) (layer B.Cu) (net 3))
 (segment (start 225.565 107.89) (end 226.59 107.89) (width 0.25) (layer F.Cu) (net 3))
 (segment (start 226.59 107.89) (end 227.055 107.425) (width 0.25) (layer F.Cu) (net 3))
 (segment (start 227.055 107.425) (end 228.295 106.185) (width 0.25) (layer B.Cu) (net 3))
 (segment (start 228.295 106.185) (end 228.295 105.355) (width 0.25) (layer B.Cu) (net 3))
 (segment (start 228.465 104.005) (end 228.465 105.185) (width 0.25) (layer F.Cu) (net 3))
 (segment (start 228.465 105.185) (end 228.295 105.355) (width 0.25) (layer F.Cu) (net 3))
 (segment (start 228.465 104.005) (end 228.465 101.935) (width 0.25) (layer B.Cu) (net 3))
 (segment (start 228.465 101.935) (end 228.485 101.915) (width 0.25) (layer B.Cu) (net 3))
 (segment (start 223.015 108.985) (end 223.995 108.985) (width 0.5) (layer F.Cu) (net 3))
 (segment (start 223.995 108.985) (end 225.09 107.89) (width 0.5) (layer F.Cu) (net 3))
 (segment (start 225.09 107.89) (end 225.565 107.89) (width 0.5) (layer F.Cu) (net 3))
 (segment (start 223.015 108.985) (end 221.085 108.985) (width 0.5) (layer F.Cu) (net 3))
 (segment (start 221.085 108.985) (end 221.075 108.995) (width 0.5) (layer F.Cu) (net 3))
 (via (at 224.225 104.925) (size 0.7) (layers F.Cu B.Cu) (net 3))
 (via (at 227.055 107.425) (size 0.7) (layers F.Cu B.Cu) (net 3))
 (via (at 228.465 104.005) (size 0.7) (layers F.Cu B.Cu) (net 3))
 (via (at 228.295 105.355) (size 0.7) (layers F.Cu B.Cu) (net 3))
 (segment (start 231.725 111.605) (end 231.885 111.605) (width 0.25) (layer B.Cu) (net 2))
 (segment (start 231.885 111.605) (end 232.705 112.425) (width 0.25) (layer B.Cu) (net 2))
 (segment (start 231.565 111.605) (end 231.725 111.605) (width 0.25) (layer B.Cu) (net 2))
 (segment (start 231.725 111.435) (end 232.005 111.435) (width 0.25) (layer B.Cu) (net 2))
 (segment (start 231.575 111.435) (end 231.725 111.435) (width 0.25) (layer B.Cu) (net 2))
 (segment (start 231.725 111.605) (end 231.725 111.435) (width 0.25) (layer B.Cu) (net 2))
 (segment (start 232.705 112.425) (end 232.705 111.815) (width 0.25) (layer F.Cu) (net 2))
 (segment (start 232.705 111.815) (end 233.485 111.035) (width 0.25) (layer F.Cu) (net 2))
 (via (at 232.705 112.425) (size 0.7) (layers F.Cu B.Cu) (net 2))
 (segment (start 221.115 111.565) (end 221.125 111.555) (width 0.25) (layer F.Cu) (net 4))
 (segment (start 221.125 111.555) (end 221.125 111.155) (width 0.25) (layer F.Cu) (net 4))
 (segment (start 221.115 111.565) (end 221.115 111.875) (width 0.25) (layer F.Cu) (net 4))
 (segment (start 221.115 111.875) (end 220.735 112.255) (width 0.25) (layer F.Cu) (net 4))
 (segment (start 221.115 111.255) (end 221.115 111.565) (width 0.25) (layer F.Cu) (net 4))
 (segment (start 220.735 112.255) (end 221.355 111.635) (width 0.25) (layer B.Cu) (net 4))
 (segment (start 221.355 111.635) (end 222.325 111.635) (width 0.25) (layer B.Cu) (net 4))
 (segment (start 222.325 111.635) (end 222.335 111.585) (width 0.25) (layer B.Cu) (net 4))
 (via (at 220.735 112.255) (size 0.7) (layers F.Cu B.Cu) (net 4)))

